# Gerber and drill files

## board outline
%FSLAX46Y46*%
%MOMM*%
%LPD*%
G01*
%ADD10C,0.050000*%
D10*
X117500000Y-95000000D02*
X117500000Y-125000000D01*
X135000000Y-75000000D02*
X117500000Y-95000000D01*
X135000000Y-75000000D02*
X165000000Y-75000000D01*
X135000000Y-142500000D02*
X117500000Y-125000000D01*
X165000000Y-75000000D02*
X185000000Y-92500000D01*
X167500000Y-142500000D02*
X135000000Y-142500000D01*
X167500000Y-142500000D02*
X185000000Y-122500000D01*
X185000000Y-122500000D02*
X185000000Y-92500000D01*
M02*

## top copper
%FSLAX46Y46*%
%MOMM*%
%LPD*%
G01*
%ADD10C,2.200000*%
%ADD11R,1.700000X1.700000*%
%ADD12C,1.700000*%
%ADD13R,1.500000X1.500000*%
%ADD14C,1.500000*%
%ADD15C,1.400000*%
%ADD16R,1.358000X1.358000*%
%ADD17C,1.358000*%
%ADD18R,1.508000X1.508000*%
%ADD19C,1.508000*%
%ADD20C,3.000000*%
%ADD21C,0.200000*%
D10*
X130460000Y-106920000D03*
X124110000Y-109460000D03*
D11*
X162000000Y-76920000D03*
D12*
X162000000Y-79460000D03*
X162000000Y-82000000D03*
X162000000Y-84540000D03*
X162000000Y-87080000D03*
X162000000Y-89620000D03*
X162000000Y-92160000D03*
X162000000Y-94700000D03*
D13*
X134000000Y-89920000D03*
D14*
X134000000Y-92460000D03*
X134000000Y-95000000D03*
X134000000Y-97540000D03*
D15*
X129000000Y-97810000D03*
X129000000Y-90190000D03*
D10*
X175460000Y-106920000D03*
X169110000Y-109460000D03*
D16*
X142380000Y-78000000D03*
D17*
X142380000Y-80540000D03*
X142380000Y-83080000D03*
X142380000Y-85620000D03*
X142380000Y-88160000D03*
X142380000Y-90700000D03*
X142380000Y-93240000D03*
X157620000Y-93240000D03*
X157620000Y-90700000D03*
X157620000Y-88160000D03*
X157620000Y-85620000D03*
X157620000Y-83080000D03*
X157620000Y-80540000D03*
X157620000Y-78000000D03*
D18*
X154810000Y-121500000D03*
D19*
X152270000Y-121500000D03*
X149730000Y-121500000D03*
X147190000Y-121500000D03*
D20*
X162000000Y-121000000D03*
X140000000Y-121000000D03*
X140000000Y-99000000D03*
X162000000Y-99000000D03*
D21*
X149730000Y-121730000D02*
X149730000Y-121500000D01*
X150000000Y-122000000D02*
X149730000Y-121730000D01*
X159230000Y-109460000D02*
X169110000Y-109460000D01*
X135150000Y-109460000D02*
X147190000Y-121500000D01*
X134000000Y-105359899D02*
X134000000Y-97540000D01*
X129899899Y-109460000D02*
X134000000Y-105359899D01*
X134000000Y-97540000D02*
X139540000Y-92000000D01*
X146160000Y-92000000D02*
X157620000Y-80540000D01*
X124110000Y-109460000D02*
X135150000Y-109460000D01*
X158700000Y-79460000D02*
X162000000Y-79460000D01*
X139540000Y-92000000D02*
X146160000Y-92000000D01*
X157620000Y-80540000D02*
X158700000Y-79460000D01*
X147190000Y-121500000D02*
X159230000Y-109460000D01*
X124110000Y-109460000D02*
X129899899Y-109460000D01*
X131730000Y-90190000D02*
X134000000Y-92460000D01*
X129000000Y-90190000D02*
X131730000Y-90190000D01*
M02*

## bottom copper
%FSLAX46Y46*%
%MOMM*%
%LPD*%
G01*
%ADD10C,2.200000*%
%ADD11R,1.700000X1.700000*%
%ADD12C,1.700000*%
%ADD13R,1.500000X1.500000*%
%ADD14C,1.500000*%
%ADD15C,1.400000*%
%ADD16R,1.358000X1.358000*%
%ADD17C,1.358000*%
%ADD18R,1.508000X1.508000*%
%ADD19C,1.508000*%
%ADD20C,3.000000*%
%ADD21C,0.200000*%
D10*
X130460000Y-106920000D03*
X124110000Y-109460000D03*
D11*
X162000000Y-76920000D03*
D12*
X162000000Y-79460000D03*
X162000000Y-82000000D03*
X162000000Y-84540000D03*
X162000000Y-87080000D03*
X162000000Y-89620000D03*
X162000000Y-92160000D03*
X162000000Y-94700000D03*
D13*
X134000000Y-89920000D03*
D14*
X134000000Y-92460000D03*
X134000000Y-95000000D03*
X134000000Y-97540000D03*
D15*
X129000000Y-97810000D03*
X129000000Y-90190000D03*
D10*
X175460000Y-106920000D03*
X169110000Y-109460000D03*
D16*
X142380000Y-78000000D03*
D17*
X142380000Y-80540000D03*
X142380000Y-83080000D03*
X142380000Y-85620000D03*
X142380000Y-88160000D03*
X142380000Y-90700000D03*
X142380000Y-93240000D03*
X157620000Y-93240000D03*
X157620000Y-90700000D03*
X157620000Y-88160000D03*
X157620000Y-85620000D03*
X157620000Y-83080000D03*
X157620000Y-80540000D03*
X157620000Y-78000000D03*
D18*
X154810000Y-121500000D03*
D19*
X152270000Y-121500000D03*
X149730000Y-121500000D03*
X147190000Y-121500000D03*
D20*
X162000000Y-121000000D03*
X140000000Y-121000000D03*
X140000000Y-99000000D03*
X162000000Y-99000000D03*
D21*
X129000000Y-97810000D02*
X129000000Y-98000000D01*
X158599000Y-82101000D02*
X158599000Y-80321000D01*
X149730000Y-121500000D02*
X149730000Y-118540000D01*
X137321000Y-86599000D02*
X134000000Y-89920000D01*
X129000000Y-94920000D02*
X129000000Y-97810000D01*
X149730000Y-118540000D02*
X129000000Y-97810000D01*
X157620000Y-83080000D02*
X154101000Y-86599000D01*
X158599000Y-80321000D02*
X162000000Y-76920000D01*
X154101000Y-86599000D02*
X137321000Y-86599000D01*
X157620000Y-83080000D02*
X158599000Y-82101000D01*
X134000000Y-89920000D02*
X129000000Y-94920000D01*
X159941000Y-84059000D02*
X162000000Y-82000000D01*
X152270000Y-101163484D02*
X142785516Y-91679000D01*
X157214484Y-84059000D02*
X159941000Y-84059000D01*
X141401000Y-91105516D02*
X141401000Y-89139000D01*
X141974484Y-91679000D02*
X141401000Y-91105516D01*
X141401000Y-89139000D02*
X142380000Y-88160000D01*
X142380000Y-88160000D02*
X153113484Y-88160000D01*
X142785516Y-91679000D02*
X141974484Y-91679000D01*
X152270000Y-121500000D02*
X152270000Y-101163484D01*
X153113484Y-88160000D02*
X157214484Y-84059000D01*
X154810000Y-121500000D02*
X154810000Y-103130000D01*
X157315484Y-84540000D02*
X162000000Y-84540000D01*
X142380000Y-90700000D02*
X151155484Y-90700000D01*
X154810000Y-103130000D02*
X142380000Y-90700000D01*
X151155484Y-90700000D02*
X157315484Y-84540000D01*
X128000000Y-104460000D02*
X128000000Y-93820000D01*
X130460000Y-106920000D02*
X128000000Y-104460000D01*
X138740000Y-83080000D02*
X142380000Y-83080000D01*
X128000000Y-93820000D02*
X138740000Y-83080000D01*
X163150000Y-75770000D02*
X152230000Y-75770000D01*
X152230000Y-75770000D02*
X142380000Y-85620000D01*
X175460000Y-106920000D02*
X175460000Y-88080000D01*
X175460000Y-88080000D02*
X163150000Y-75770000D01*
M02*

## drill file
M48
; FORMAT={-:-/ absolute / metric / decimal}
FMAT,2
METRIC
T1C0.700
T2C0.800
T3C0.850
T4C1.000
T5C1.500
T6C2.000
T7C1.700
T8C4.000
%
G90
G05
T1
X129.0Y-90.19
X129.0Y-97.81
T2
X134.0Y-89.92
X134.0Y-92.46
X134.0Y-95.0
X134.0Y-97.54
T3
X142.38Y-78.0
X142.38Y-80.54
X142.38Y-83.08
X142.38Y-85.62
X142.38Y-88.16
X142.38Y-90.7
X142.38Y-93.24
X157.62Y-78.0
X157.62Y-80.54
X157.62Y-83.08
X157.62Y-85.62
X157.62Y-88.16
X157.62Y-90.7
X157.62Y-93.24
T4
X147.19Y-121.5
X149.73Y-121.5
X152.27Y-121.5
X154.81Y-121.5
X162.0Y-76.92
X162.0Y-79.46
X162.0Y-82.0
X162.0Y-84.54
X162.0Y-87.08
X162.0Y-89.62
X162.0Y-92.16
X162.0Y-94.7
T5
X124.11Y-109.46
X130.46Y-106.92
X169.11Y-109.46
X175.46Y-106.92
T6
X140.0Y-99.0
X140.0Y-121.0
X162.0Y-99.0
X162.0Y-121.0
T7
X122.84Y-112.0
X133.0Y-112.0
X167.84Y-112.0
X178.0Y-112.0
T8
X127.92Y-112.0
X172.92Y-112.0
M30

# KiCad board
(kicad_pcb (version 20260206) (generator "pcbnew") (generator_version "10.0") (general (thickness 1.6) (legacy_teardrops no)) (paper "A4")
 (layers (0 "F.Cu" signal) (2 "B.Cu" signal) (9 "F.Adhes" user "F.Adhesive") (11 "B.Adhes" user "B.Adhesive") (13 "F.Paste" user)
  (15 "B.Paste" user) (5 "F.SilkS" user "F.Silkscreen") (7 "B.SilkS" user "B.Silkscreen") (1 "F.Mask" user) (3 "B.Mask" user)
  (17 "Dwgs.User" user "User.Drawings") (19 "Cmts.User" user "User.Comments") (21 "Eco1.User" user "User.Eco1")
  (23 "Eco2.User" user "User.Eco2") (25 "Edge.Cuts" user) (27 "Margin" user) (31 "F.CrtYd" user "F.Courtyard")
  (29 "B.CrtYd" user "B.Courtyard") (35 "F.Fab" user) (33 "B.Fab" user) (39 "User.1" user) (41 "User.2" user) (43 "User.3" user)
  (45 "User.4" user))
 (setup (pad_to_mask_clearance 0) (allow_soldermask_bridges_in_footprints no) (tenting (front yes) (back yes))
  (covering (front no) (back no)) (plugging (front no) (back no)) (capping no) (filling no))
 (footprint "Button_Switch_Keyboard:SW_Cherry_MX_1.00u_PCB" (layer "F.Cu") (at 130.46 106.92)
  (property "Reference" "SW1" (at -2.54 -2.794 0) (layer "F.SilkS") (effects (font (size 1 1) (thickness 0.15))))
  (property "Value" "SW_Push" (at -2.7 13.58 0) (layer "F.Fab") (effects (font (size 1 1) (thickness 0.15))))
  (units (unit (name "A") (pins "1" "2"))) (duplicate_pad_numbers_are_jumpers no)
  (pad "" np_thru_hole circle (at -7.62 5.08) (size 1.7 1.7) (drill 1.7) (layers "*.Cu" "*.Mask"))
  (pad "" np_thru_hole circle (at -2.54 5.08) (size 4 4) (drill 4) (layers "*.Cu" "*.Mask"))
  (pad "" np_thru_hole circle (at 2.54 5.08) (size 1.7 1.7) (drill 1.7) (layers "*.Cu" "*.Mask"))
  (pad "1" thru_hole circle (at 0 0) (size 2.2 2.2) (drill 1.5) (layers "*.Cu" "*.Mask") (remove_unused_layers no) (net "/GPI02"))
  (pad "2" thru_hole circle (at -6.35 2.54) (size 2.2 2.2) (drill 1.5) (layers "*.Cu" "*.Mask") (remove_unused_layers no) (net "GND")))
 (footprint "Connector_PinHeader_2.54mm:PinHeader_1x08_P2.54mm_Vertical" (layer "F.Cu") (at 162 76.92)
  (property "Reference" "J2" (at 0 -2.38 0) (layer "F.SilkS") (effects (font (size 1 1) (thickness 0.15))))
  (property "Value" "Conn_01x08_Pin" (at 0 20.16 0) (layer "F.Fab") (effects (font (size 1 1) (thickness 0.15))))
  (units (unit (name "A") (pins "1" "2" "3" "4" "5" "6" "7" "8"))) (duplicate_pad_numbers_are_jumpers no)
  (pad "1" thru_hole rect (at 0 0) (size 1.7 1.7) (drill 1) (layers "*.Cu" "*.Mask") (remove_unused_layers no) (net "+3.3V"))
  (pad "2" thru_hole circle (at 0 2.54) (size 1.7 1.7) (drill 1) (layers "*.Cu" "*.Mask") (remove_unused_layers no) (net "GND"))
  (pad "3" thru_hole circle (at 0 5.08) (size 1.7 1.7) (drill 1) (layers "*.Cu" "*.Mask") (remove_unused_layers no) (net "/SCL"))
  (pad "4" thru_hole circle (at 0 7.62) (size 1.7 1.7) (drill 1) (layers "*.Cu" "*.Mask") (remove_unused_layers no) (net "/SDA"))
  (pad "5" thru_hole circle (at 0 10.16) (size 1.7 1.7) (drill 1) (layers "*.Cu" "*.Mask") (remove_unused_layers no)
   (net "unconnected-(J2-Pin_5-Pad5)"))
  (pad "6" thru_hole circle (at 0 12.7) (size 1.7 1.7) (drill 1) (layers "*.Cu" "*.Mask") (remove_unused_layers no)
   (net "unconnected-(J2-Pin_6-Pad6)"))
  (pad "7" thru_hole circle (at 0 15.24) (size 1.7 1.7) (drill 1) (layers "*.Cu" "*.Mask") (remove_unused_layers no)
   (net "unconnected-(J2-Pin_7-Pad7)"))
  (pad "8" thru_hole circle (at 0 17.78) (size 1.7 1.7) (drill 1) (layers "*.Cu" "*.Mask") (remove_unused_layers no)
   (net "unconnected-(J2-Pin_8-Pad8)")))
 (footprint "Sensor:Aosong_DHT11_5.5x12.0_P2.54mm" (layer "F.Cu") (at 134 89.92)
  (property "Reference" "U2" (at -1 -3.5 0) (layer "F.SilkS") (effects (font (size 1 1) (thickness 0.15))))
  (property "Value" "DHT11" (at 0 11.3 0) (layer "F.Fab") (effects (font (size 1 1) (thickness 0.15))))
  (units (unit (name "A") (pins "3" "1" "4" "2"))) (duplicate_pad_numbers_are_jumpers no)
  (pad "1" thru_hole rect (at 0 0) (size 1.5 1.5) (drill 0.8) (layers "*.Cu" "*.Mask") (remove_unused_layers no) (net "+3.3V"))
  (pad "2" thru_hole circle (at 0 2.54) (size 1.5 1.5) (drill 0.8) (layers "*.Cu" "*.Mask") (remove_unused_layers no) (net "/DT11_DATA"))
  (pad "3" thru_hole circle (at 0 5.08) (size 1.5 1.5) (drill 0.8) (layers "*.Cu" "*.Mask") (remove_unused_layers no)
   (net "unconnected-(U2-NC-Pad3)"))
  (pad "4" thru_hole circle (at 0 7.62) (size 1.5 1.5) (drill 0.8) (layers "*.Cu" "*.Mask") (remove_unused_layers no) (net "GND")))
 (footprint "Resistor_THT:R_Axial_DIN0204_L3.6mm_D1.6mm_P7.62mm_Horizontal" (layer "F.Cu") (at 129 97.81 90)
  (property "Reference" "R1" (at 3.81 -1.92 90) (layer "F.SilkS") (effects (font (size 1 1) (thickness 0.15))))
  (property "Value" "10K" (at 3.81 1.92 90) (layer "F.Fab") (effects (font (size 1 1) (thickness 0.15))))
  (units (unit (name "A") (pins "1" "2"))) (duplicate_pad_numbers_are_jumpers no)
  (pad "1" thru_hole circle (at 0 0 90) (size 1.4 1.4) (drill 0.7) (layers "*.Cu" "*.Mask") (remove_unused_layers no) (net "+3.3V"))
  (pad "2" thru_hole circle (at 7.62 0 90) (size 1.4 1.4) (drill 0.7) (layers "*.Cu" "*.Mask") (remove_unused_layers no) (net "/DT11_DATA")))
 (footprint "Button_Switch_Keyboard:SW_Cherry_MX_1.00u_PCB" (layer "F.Cu") (at 175.46 106.92)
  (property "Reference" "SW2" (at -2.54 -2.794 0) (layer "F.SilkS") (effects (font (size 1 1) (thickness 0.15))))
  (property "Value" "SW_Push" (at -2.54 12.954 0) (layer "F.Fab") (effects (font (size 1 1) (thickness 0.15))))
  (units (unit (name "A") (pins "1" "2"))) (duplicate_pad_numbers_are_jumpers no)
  (pad "" np_thru_hole circle (at -7.62 5.08) (size 1.7 1.7) (drill 1.7) (layers "*.Cu" "*.Mask"))
  (pad "" np_thru_hole circle (at -2.54 5.08) (size 4 4) (drill 4) (layers "*.Cu" "*.Mask"))
  (pad "" np_thru_hole circle (at 2.54 5.08) (size 1.7 1.7) (drill 1.7) (layers "*.Cu" "*.Mask"))
  (pad "1" thru_hole circle (at 0 0) (size 2.2 2.2) (drill 1.5) (layers "*.Cu" "*.Mask") (remove_unused_layers no) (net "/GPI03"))
  (pad "2" thru_hole circle (at -6.35 2.54) (size 2.2 2.2) (drill 1.5) (layers "*.Cu" "*.Mask") (remove_unused_layers no) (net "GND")))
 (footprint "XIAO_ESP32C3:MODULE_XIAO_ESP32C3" (layer "F.Cu") (at 150 85.5565)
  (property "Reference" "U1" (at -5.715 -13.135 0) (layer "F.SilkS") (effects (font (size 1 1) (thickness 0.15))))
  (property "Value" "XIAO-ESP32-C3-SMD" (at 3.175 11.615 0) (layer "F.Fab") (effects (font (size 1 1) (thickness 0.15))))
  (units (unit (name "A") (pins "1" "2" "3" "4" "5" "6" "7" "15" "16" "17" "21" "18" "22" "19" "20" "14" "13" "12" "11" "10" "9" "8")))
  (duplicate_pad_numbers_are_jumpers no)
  (pad "1" thru_hole rect (at -7.62 -7.5565) (size 1.358 1.358) (drill 0.85) (layers "*.Cu" "*.Mask") (remove_unused_layers no)
   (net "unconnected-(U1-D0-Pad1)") (solder_mask_margin 0.102))
  (pad "2" thru_hole circle (at -7.62 -5.0165) (size 1.358 1.358) (drill 0.85) (layers "*.Cu" "*.Mask") (remove_unused_layers no)
   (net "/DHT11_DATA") (solder_mask_margin 0.102))
  (pad "3" thru_hole circle (at -7.62 -2.4765) (size 1.358 1.358) (drill 0.85) (layers "*.Cu" "*.Mask") (remove_unused_layers no)
   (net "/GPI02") (solder_mask_margin 0.102))
  (pad "4" thru_hole circle (at -7.62 0.0635) (size 1.358 1.358) (drill 0.85) (layers "*.Cu" "*.Mask") (remove_unused_layers no)
   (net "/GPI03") (solder_mask_margin 0.102))
  (pad "5" thru_hole circle (at -7.62 2.6035) (size 1.358 1.358) (drill 0.85) (layers "*.Cu" "*.Mask") (remove_unused_layers no)
   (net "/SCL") (solder_mask_margin 0.102))
  (pad "6" thru_hole circle (at -7.62 5.1435) (size 1.358 1.358) (drill 0.85) (layers "*.Cu" "*.Mask") (remove_unused_layers no)
   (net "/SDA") (solder_mask_margin 0.102))
  (pad "7" thru_hole circle (at -7.62 7.6835) (size 1.358 1.358) (drill 0.85) (layers "*.Cu" "*.Mask") (remove_unused_layers no)
   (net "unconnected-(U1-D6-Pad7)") (solder_mask_margin 0.102))
  (pad "8" thru_hole circle (at 7.62 7.6835) (size 1.358 1.358) (drill 0.85) (layers "*.Cu" "*.Mask") (remove_unused_layers no)
   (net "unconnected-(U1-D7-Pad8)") (solder_mask_margin 0.102))
  (pad "9" thru_hole circle (at 7.62 5.1435) (size 1.358 1.358) (drill 0.85) (layers "*.Cu" "*.Mask") (remove_unused_layers no)
   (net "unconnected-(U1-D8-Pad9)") (solder_mask_margin 0.102))
  (pad "10" thru_hole circle (at 7.62 2.6035) (size 1.358 1.358) (drill 0.85) (layers "*.Cu" "*.Mask") (remove_unused_layers no)
   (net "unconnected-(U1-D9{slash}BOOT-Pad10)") (solder_mask_margin 0.102))
  (pad "11" thru_hole circle (at 7.62 0.0635) (size 1.358 1.358) (drill 0.85) (layers "*.Cu" "*.Mask") (remove_unused_layers no)
   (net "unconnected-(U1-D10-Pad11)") (solder_mask_margin 0.102))
  (pad "12" thru_hole circle (at 7.62 -2.4765) (size 1.358 1.358) (drill 0.85) (layers "*.Cu" "*.Mask") (remove_unused_layers no)
   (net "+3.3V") (solder_mask_margin 0.102))
  (pad "13" thru_hole circle (at 7.62 -5.0165) (size 1.358 1.358) (drill 0.85) (layers "*.Cu" "*.Mask") (remove_unused_layers no)
   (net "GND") (solder_mask_margin 0.102))
  (pad "14" thru_hole circle (at 7.62 -7.5565) (size 1.358 1.358) (drill 0.85) (layers "*.Cu" "*.Mask") (remove_unused_layers no)
   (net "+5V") (solder_mask_margin 0.102)))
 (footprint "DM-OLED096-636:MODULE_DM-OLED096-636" (layer "F.Cu") (at 151 110 180)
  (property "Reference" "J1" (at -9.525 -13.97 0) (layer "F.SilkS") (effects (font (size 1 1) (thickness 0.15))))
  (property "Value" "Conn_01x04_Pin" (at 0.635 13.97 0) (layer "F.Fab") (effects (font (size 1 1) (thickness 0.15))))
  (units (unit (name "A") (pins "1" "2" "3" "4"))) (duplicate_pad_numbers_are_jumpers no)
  (pad "1" thru_hole rect (at -3.81 -11.5 180) (size 1.508 1.508) (drill 1) (layers "*.Cu" "*.Mask") (remove_unused_layers no) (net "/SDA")
   (solder_mask_margin 0.102))
  (pad "2" thru_hole circle (at -1.27 -11.5 180) (size 1.508 1.508) (drill 1) (layers "*.Cu" "*.Mask") (remove_unused_layers no)
   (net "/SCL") (solder_mask_margin 0.102))
  (pad "3" thru_hole circle (at 1.27 -11.5 180) (size 1.508 1.508) (drill 1) (layers "*.Cu" "*.Mask") (remove_unused_layers no)
   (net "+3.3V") (solder_mask_margin 0.102))
  (pad "4" thru_hole circle (at 3.81 -11.5 180) (size 1.508 1.508) (drill 1) (layers "*.Cu" "*.Mask") (remove_unused_layers no) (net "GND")
   (solder_mask_margin 0.102))
  (pad "S1" thru_hole circle (at -11 -11 180) (size 3 3) (drill 2) (layers "*.Cu" "*.Mask") (remove_unused_layers no)
   (solder_mask_margin 0.102))
  (pad "S2" thru_hole circle (at 11 -11 180) (size 3 3) (drill 2) (layers "*.Cu" "*.Mask") (remove_unused_layers no)
   (solder_mask_margin 0.102))
  (pad "S3" thru_hole circle (at 11 11 180) (size 3 3) (drill 2) (layers "*.Cu" "*.Mask") (remove_unused_layers no)
   (solder_mask_margin 0.102))
  (pad "S4" thru_hole circle (at -11 11 180) (size 3 3) (drill 2) (layers "*.Cu" "*.Mask") (remove_unused_layers no)
   (solder_mask_margin 0.102)))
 (gr_line (start 117.5 95) (end 117.5 125) (stroke (width 0.05) (type default)) (layer "Edge.Cuts"))
 (gr_line (start 135 75) (end 117.5 95) (stroke (width 0.05) (type default)) (layer "Edge.Cuts"))
 (gr_line (start 135 75) (end 165 75) (stroke (width 0.05) (type default)) (layer "Edge.Cuts"))
 (gr_line (start 135 142.5) (end 117.5 125) (stroke (width 0.05) (type default)) (layer "Edge.Cuts"))
 (gr_line (start 165 75) (end 185 92.5) (stroke (width 0.05) (type default)) (layer "Edge.Cuts"))
 (gr_line (start 167.5 142.5) (end 135 142.5) (stroke (width 0.05) (type default)) (layer "Edge.Cuts"))
 (gr_line (start 167.5 142.5) (end 185 122.5) (stroke (width 0.05) (type default)) (layer "Edge.Cuts"))
 (gr_line (start 185 122.5) (end 185 92.5) (stroke (width 0.05) (type default)) (layer "Edge.Cuts"))
 (segment (start 149.73 121.73) (end 149.73 121.5) (width 0.2) (layer "F.Cu") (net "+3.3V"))
 (segment (start 150 122) (end 149.73 121.73) (width 0.2) (layer "F.Cu") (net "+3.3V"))
 (segment (start 129 97.81) (end 129 98) (width 0.2) (layer "B.Cu") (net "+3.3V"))
 (segment (start 158.599 82.101) (end 158.599 80.321) (width 0.2) (layer "B.Cu") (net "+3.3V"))
 (segment (start 149.73 121.5) (end 149.73 118.54) (width 0.2) (layer "B.Cu") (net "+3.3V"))
 (segment (start 137.321 86.599) (end 134 89.92) (width 0.2) (layer "B.Cu") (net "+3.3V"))
 (segment (start 129 94.92) (end 129 97.81) (width 0.2) (layer "B.Cu") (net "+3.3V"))
 (segment (start 149.73 118.54) (end 129 97.81) (width 0.2) (layer "B.Cu") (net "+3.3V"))
 (segment (start 157.62 83.08) (end 154.101 86.599) (width 0.2) (layer "B.Cu") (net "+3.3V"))
 (segment (start 158.599 80.321) (end 162 76.92) (width 0.2) (layer "B.Cu") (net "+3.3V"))
 (segment (start 154.101 86.599) (end 137.321 86.599) (width 0.2) (layer "B.Cu") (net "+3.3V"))
 (segment (start 157.62 83.08) (end 158.599 82.101) (width 0.2) (layer "B.Cu") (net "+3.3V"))
 (segment (start 134 89.92) (end 129 94.92) (width 0.2) (layer "B.Cu") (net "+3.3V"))
 (segment (start 159.23 109.46) (end 169.11 109.46) (width 0.2) (layer "F.Cu") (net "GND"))
 (segment (start 135.15 109.46) (end 147.19 121.5) (width 0.2) (layer "F.Cu") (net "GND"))
 (segment (start 134 105.359899) (end 134 97.54) (width 0.2) (layer "F.Cu") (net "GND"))
 (segment (start 129.899899 109.46) (end 134 105.359899) (width 0.2) (layer "F.Cu") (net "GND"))
 (segment (start 134 97.54) (end 139.54 92) (width 0.2) (layer "F.Cu") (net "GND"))
 (segment (start 146.16 92) (end 157.62 80.54) (width 0.2) (layer "F.Cu") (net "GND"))
 (segment (start 124.11 109.46) (end 135.15 109.46) (width 0.2) (layer "F.Cu") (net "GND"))
 (segment (start 158.7 79.46) (end 162 79.46) (width 0.2) (layer "F.Cu") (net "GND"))
 (segment (start 139.54 92) (end 146.16 92) (width 0.2) (layer "F.Cu") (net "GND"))
 (segment (start 157.62 80.54) (end 158.7 79.46) (width 0.2) (layer "F.Cu") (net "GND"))
 (segment (start 147.19 121.5) (end 159.23 109.46) (width 0.2) (layer "F.Cu") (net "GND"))
 (segment (start 124.11 109.46) (end 129.899899 109.46) (width 0.2) (layer "F.Cu") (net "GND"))
 (segment (start 159.941 84.059) (end 162 82) (width 0.2) (layer "B.Cu") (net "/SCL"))
 (segment (start 152.27 101.163484) (end 142.785516 91.679) (width 0.2) (layer "B.Cu") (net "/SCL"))
 (segment (start 157.214484 84.059) (end 159.941 84.059) (width 0.2) (layer "B.Cu") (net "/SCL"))
 (segment (start 141.401 91.105516) (end 141.401 89.139) (width 0.2) (layer "B.Cu") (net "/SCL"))
 (segment (start 141.974484 91.679) (end 141.401 91.105516) (width 0.2) (layer "B.Cu") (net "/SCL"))
 (segment (start 141.401 89.139) (end 142.38 88.16) (width 0.2) (layer "B.Cu") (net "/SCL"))
 (segment (start 142.38 88.16) (end 153.113484 88.16) (width 0.2) (layer "B.Cu") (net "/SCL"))
 (segment (start 142.785516 91.679) (end 141.974484 91.679) (width 0.2) (layer "B.Cu") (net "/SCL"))
 (segment (start 152.27 121.5) (end 152.27 101.163484) (width 0.2) (layer "B.Cu") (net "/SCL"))
 (segment (start 153.113484 88.16) (end 157.214484 84.059) (width 0.2) (layer "B.Cu") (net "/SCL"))
 (segment (start 154.81 121.5) (end 154.81 103.13) (width 0.2) (layer "B.Cu") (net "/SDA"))
 (segment (start 157.315484 84.54) (end 162 84.54) (width 0.2) (layer "B.Cu") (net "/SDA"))
 (segment (start 142.38 90.7) (end 151.155484 90.7) (width 0.2) (layer "B.Cu") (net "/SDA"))
 (segment (start 154.81 103.13) (end 142.38 90.7) (width 0.2) (layer "B.Cu") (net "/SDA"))
 (segment (start 151.155484 90.7) (end 157.315484 84.54) (width 0.2) (layer "B.Cu") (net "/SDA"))
 (segment (start 131.73 90.19) (end 134 92.46) (width 0.2) (layer "F.Cu") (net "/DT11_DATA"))
 (segment (start 129 90.19) (end 131.73 90.19) (width 0.2) (layer "F.Cu") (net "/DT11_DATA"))
 (segment (start 128 104.46) (end 128 93.82) (width 0.2) (layer "B.Cu") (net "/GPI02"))
 (segment (start 130.46 106.92) (end 128 104.46) (width 0.2) (layer "B.Cu") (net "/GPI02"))
 (segment (start 138.74 83.08) (end 142.38 83.08) (width 0.2) (layer "B.Cu") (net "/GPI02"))
 (segment (start 128 93.82) (end 138.74 83.08) (width 0.2) (layer "B.Cu") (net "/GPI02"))
 (segment (start 163.15 75.77) (end 152.23 75.77) (width 0.2) (layer "B.Cu") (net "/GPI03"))
 (segment (start 152.23 75.77) (end 142.38 85.62) (width 0.2) (layer "B.Cu") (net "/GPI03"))
 (segment (start 175.46 106.92) (end 175.46 88.08) (width 0.2) (layer "B.Cu") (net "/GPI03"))
 (segment (start 175.46 88.08) (end 163.15 75.77) (width 0.2) (layer "B.Cu") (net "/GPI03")))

